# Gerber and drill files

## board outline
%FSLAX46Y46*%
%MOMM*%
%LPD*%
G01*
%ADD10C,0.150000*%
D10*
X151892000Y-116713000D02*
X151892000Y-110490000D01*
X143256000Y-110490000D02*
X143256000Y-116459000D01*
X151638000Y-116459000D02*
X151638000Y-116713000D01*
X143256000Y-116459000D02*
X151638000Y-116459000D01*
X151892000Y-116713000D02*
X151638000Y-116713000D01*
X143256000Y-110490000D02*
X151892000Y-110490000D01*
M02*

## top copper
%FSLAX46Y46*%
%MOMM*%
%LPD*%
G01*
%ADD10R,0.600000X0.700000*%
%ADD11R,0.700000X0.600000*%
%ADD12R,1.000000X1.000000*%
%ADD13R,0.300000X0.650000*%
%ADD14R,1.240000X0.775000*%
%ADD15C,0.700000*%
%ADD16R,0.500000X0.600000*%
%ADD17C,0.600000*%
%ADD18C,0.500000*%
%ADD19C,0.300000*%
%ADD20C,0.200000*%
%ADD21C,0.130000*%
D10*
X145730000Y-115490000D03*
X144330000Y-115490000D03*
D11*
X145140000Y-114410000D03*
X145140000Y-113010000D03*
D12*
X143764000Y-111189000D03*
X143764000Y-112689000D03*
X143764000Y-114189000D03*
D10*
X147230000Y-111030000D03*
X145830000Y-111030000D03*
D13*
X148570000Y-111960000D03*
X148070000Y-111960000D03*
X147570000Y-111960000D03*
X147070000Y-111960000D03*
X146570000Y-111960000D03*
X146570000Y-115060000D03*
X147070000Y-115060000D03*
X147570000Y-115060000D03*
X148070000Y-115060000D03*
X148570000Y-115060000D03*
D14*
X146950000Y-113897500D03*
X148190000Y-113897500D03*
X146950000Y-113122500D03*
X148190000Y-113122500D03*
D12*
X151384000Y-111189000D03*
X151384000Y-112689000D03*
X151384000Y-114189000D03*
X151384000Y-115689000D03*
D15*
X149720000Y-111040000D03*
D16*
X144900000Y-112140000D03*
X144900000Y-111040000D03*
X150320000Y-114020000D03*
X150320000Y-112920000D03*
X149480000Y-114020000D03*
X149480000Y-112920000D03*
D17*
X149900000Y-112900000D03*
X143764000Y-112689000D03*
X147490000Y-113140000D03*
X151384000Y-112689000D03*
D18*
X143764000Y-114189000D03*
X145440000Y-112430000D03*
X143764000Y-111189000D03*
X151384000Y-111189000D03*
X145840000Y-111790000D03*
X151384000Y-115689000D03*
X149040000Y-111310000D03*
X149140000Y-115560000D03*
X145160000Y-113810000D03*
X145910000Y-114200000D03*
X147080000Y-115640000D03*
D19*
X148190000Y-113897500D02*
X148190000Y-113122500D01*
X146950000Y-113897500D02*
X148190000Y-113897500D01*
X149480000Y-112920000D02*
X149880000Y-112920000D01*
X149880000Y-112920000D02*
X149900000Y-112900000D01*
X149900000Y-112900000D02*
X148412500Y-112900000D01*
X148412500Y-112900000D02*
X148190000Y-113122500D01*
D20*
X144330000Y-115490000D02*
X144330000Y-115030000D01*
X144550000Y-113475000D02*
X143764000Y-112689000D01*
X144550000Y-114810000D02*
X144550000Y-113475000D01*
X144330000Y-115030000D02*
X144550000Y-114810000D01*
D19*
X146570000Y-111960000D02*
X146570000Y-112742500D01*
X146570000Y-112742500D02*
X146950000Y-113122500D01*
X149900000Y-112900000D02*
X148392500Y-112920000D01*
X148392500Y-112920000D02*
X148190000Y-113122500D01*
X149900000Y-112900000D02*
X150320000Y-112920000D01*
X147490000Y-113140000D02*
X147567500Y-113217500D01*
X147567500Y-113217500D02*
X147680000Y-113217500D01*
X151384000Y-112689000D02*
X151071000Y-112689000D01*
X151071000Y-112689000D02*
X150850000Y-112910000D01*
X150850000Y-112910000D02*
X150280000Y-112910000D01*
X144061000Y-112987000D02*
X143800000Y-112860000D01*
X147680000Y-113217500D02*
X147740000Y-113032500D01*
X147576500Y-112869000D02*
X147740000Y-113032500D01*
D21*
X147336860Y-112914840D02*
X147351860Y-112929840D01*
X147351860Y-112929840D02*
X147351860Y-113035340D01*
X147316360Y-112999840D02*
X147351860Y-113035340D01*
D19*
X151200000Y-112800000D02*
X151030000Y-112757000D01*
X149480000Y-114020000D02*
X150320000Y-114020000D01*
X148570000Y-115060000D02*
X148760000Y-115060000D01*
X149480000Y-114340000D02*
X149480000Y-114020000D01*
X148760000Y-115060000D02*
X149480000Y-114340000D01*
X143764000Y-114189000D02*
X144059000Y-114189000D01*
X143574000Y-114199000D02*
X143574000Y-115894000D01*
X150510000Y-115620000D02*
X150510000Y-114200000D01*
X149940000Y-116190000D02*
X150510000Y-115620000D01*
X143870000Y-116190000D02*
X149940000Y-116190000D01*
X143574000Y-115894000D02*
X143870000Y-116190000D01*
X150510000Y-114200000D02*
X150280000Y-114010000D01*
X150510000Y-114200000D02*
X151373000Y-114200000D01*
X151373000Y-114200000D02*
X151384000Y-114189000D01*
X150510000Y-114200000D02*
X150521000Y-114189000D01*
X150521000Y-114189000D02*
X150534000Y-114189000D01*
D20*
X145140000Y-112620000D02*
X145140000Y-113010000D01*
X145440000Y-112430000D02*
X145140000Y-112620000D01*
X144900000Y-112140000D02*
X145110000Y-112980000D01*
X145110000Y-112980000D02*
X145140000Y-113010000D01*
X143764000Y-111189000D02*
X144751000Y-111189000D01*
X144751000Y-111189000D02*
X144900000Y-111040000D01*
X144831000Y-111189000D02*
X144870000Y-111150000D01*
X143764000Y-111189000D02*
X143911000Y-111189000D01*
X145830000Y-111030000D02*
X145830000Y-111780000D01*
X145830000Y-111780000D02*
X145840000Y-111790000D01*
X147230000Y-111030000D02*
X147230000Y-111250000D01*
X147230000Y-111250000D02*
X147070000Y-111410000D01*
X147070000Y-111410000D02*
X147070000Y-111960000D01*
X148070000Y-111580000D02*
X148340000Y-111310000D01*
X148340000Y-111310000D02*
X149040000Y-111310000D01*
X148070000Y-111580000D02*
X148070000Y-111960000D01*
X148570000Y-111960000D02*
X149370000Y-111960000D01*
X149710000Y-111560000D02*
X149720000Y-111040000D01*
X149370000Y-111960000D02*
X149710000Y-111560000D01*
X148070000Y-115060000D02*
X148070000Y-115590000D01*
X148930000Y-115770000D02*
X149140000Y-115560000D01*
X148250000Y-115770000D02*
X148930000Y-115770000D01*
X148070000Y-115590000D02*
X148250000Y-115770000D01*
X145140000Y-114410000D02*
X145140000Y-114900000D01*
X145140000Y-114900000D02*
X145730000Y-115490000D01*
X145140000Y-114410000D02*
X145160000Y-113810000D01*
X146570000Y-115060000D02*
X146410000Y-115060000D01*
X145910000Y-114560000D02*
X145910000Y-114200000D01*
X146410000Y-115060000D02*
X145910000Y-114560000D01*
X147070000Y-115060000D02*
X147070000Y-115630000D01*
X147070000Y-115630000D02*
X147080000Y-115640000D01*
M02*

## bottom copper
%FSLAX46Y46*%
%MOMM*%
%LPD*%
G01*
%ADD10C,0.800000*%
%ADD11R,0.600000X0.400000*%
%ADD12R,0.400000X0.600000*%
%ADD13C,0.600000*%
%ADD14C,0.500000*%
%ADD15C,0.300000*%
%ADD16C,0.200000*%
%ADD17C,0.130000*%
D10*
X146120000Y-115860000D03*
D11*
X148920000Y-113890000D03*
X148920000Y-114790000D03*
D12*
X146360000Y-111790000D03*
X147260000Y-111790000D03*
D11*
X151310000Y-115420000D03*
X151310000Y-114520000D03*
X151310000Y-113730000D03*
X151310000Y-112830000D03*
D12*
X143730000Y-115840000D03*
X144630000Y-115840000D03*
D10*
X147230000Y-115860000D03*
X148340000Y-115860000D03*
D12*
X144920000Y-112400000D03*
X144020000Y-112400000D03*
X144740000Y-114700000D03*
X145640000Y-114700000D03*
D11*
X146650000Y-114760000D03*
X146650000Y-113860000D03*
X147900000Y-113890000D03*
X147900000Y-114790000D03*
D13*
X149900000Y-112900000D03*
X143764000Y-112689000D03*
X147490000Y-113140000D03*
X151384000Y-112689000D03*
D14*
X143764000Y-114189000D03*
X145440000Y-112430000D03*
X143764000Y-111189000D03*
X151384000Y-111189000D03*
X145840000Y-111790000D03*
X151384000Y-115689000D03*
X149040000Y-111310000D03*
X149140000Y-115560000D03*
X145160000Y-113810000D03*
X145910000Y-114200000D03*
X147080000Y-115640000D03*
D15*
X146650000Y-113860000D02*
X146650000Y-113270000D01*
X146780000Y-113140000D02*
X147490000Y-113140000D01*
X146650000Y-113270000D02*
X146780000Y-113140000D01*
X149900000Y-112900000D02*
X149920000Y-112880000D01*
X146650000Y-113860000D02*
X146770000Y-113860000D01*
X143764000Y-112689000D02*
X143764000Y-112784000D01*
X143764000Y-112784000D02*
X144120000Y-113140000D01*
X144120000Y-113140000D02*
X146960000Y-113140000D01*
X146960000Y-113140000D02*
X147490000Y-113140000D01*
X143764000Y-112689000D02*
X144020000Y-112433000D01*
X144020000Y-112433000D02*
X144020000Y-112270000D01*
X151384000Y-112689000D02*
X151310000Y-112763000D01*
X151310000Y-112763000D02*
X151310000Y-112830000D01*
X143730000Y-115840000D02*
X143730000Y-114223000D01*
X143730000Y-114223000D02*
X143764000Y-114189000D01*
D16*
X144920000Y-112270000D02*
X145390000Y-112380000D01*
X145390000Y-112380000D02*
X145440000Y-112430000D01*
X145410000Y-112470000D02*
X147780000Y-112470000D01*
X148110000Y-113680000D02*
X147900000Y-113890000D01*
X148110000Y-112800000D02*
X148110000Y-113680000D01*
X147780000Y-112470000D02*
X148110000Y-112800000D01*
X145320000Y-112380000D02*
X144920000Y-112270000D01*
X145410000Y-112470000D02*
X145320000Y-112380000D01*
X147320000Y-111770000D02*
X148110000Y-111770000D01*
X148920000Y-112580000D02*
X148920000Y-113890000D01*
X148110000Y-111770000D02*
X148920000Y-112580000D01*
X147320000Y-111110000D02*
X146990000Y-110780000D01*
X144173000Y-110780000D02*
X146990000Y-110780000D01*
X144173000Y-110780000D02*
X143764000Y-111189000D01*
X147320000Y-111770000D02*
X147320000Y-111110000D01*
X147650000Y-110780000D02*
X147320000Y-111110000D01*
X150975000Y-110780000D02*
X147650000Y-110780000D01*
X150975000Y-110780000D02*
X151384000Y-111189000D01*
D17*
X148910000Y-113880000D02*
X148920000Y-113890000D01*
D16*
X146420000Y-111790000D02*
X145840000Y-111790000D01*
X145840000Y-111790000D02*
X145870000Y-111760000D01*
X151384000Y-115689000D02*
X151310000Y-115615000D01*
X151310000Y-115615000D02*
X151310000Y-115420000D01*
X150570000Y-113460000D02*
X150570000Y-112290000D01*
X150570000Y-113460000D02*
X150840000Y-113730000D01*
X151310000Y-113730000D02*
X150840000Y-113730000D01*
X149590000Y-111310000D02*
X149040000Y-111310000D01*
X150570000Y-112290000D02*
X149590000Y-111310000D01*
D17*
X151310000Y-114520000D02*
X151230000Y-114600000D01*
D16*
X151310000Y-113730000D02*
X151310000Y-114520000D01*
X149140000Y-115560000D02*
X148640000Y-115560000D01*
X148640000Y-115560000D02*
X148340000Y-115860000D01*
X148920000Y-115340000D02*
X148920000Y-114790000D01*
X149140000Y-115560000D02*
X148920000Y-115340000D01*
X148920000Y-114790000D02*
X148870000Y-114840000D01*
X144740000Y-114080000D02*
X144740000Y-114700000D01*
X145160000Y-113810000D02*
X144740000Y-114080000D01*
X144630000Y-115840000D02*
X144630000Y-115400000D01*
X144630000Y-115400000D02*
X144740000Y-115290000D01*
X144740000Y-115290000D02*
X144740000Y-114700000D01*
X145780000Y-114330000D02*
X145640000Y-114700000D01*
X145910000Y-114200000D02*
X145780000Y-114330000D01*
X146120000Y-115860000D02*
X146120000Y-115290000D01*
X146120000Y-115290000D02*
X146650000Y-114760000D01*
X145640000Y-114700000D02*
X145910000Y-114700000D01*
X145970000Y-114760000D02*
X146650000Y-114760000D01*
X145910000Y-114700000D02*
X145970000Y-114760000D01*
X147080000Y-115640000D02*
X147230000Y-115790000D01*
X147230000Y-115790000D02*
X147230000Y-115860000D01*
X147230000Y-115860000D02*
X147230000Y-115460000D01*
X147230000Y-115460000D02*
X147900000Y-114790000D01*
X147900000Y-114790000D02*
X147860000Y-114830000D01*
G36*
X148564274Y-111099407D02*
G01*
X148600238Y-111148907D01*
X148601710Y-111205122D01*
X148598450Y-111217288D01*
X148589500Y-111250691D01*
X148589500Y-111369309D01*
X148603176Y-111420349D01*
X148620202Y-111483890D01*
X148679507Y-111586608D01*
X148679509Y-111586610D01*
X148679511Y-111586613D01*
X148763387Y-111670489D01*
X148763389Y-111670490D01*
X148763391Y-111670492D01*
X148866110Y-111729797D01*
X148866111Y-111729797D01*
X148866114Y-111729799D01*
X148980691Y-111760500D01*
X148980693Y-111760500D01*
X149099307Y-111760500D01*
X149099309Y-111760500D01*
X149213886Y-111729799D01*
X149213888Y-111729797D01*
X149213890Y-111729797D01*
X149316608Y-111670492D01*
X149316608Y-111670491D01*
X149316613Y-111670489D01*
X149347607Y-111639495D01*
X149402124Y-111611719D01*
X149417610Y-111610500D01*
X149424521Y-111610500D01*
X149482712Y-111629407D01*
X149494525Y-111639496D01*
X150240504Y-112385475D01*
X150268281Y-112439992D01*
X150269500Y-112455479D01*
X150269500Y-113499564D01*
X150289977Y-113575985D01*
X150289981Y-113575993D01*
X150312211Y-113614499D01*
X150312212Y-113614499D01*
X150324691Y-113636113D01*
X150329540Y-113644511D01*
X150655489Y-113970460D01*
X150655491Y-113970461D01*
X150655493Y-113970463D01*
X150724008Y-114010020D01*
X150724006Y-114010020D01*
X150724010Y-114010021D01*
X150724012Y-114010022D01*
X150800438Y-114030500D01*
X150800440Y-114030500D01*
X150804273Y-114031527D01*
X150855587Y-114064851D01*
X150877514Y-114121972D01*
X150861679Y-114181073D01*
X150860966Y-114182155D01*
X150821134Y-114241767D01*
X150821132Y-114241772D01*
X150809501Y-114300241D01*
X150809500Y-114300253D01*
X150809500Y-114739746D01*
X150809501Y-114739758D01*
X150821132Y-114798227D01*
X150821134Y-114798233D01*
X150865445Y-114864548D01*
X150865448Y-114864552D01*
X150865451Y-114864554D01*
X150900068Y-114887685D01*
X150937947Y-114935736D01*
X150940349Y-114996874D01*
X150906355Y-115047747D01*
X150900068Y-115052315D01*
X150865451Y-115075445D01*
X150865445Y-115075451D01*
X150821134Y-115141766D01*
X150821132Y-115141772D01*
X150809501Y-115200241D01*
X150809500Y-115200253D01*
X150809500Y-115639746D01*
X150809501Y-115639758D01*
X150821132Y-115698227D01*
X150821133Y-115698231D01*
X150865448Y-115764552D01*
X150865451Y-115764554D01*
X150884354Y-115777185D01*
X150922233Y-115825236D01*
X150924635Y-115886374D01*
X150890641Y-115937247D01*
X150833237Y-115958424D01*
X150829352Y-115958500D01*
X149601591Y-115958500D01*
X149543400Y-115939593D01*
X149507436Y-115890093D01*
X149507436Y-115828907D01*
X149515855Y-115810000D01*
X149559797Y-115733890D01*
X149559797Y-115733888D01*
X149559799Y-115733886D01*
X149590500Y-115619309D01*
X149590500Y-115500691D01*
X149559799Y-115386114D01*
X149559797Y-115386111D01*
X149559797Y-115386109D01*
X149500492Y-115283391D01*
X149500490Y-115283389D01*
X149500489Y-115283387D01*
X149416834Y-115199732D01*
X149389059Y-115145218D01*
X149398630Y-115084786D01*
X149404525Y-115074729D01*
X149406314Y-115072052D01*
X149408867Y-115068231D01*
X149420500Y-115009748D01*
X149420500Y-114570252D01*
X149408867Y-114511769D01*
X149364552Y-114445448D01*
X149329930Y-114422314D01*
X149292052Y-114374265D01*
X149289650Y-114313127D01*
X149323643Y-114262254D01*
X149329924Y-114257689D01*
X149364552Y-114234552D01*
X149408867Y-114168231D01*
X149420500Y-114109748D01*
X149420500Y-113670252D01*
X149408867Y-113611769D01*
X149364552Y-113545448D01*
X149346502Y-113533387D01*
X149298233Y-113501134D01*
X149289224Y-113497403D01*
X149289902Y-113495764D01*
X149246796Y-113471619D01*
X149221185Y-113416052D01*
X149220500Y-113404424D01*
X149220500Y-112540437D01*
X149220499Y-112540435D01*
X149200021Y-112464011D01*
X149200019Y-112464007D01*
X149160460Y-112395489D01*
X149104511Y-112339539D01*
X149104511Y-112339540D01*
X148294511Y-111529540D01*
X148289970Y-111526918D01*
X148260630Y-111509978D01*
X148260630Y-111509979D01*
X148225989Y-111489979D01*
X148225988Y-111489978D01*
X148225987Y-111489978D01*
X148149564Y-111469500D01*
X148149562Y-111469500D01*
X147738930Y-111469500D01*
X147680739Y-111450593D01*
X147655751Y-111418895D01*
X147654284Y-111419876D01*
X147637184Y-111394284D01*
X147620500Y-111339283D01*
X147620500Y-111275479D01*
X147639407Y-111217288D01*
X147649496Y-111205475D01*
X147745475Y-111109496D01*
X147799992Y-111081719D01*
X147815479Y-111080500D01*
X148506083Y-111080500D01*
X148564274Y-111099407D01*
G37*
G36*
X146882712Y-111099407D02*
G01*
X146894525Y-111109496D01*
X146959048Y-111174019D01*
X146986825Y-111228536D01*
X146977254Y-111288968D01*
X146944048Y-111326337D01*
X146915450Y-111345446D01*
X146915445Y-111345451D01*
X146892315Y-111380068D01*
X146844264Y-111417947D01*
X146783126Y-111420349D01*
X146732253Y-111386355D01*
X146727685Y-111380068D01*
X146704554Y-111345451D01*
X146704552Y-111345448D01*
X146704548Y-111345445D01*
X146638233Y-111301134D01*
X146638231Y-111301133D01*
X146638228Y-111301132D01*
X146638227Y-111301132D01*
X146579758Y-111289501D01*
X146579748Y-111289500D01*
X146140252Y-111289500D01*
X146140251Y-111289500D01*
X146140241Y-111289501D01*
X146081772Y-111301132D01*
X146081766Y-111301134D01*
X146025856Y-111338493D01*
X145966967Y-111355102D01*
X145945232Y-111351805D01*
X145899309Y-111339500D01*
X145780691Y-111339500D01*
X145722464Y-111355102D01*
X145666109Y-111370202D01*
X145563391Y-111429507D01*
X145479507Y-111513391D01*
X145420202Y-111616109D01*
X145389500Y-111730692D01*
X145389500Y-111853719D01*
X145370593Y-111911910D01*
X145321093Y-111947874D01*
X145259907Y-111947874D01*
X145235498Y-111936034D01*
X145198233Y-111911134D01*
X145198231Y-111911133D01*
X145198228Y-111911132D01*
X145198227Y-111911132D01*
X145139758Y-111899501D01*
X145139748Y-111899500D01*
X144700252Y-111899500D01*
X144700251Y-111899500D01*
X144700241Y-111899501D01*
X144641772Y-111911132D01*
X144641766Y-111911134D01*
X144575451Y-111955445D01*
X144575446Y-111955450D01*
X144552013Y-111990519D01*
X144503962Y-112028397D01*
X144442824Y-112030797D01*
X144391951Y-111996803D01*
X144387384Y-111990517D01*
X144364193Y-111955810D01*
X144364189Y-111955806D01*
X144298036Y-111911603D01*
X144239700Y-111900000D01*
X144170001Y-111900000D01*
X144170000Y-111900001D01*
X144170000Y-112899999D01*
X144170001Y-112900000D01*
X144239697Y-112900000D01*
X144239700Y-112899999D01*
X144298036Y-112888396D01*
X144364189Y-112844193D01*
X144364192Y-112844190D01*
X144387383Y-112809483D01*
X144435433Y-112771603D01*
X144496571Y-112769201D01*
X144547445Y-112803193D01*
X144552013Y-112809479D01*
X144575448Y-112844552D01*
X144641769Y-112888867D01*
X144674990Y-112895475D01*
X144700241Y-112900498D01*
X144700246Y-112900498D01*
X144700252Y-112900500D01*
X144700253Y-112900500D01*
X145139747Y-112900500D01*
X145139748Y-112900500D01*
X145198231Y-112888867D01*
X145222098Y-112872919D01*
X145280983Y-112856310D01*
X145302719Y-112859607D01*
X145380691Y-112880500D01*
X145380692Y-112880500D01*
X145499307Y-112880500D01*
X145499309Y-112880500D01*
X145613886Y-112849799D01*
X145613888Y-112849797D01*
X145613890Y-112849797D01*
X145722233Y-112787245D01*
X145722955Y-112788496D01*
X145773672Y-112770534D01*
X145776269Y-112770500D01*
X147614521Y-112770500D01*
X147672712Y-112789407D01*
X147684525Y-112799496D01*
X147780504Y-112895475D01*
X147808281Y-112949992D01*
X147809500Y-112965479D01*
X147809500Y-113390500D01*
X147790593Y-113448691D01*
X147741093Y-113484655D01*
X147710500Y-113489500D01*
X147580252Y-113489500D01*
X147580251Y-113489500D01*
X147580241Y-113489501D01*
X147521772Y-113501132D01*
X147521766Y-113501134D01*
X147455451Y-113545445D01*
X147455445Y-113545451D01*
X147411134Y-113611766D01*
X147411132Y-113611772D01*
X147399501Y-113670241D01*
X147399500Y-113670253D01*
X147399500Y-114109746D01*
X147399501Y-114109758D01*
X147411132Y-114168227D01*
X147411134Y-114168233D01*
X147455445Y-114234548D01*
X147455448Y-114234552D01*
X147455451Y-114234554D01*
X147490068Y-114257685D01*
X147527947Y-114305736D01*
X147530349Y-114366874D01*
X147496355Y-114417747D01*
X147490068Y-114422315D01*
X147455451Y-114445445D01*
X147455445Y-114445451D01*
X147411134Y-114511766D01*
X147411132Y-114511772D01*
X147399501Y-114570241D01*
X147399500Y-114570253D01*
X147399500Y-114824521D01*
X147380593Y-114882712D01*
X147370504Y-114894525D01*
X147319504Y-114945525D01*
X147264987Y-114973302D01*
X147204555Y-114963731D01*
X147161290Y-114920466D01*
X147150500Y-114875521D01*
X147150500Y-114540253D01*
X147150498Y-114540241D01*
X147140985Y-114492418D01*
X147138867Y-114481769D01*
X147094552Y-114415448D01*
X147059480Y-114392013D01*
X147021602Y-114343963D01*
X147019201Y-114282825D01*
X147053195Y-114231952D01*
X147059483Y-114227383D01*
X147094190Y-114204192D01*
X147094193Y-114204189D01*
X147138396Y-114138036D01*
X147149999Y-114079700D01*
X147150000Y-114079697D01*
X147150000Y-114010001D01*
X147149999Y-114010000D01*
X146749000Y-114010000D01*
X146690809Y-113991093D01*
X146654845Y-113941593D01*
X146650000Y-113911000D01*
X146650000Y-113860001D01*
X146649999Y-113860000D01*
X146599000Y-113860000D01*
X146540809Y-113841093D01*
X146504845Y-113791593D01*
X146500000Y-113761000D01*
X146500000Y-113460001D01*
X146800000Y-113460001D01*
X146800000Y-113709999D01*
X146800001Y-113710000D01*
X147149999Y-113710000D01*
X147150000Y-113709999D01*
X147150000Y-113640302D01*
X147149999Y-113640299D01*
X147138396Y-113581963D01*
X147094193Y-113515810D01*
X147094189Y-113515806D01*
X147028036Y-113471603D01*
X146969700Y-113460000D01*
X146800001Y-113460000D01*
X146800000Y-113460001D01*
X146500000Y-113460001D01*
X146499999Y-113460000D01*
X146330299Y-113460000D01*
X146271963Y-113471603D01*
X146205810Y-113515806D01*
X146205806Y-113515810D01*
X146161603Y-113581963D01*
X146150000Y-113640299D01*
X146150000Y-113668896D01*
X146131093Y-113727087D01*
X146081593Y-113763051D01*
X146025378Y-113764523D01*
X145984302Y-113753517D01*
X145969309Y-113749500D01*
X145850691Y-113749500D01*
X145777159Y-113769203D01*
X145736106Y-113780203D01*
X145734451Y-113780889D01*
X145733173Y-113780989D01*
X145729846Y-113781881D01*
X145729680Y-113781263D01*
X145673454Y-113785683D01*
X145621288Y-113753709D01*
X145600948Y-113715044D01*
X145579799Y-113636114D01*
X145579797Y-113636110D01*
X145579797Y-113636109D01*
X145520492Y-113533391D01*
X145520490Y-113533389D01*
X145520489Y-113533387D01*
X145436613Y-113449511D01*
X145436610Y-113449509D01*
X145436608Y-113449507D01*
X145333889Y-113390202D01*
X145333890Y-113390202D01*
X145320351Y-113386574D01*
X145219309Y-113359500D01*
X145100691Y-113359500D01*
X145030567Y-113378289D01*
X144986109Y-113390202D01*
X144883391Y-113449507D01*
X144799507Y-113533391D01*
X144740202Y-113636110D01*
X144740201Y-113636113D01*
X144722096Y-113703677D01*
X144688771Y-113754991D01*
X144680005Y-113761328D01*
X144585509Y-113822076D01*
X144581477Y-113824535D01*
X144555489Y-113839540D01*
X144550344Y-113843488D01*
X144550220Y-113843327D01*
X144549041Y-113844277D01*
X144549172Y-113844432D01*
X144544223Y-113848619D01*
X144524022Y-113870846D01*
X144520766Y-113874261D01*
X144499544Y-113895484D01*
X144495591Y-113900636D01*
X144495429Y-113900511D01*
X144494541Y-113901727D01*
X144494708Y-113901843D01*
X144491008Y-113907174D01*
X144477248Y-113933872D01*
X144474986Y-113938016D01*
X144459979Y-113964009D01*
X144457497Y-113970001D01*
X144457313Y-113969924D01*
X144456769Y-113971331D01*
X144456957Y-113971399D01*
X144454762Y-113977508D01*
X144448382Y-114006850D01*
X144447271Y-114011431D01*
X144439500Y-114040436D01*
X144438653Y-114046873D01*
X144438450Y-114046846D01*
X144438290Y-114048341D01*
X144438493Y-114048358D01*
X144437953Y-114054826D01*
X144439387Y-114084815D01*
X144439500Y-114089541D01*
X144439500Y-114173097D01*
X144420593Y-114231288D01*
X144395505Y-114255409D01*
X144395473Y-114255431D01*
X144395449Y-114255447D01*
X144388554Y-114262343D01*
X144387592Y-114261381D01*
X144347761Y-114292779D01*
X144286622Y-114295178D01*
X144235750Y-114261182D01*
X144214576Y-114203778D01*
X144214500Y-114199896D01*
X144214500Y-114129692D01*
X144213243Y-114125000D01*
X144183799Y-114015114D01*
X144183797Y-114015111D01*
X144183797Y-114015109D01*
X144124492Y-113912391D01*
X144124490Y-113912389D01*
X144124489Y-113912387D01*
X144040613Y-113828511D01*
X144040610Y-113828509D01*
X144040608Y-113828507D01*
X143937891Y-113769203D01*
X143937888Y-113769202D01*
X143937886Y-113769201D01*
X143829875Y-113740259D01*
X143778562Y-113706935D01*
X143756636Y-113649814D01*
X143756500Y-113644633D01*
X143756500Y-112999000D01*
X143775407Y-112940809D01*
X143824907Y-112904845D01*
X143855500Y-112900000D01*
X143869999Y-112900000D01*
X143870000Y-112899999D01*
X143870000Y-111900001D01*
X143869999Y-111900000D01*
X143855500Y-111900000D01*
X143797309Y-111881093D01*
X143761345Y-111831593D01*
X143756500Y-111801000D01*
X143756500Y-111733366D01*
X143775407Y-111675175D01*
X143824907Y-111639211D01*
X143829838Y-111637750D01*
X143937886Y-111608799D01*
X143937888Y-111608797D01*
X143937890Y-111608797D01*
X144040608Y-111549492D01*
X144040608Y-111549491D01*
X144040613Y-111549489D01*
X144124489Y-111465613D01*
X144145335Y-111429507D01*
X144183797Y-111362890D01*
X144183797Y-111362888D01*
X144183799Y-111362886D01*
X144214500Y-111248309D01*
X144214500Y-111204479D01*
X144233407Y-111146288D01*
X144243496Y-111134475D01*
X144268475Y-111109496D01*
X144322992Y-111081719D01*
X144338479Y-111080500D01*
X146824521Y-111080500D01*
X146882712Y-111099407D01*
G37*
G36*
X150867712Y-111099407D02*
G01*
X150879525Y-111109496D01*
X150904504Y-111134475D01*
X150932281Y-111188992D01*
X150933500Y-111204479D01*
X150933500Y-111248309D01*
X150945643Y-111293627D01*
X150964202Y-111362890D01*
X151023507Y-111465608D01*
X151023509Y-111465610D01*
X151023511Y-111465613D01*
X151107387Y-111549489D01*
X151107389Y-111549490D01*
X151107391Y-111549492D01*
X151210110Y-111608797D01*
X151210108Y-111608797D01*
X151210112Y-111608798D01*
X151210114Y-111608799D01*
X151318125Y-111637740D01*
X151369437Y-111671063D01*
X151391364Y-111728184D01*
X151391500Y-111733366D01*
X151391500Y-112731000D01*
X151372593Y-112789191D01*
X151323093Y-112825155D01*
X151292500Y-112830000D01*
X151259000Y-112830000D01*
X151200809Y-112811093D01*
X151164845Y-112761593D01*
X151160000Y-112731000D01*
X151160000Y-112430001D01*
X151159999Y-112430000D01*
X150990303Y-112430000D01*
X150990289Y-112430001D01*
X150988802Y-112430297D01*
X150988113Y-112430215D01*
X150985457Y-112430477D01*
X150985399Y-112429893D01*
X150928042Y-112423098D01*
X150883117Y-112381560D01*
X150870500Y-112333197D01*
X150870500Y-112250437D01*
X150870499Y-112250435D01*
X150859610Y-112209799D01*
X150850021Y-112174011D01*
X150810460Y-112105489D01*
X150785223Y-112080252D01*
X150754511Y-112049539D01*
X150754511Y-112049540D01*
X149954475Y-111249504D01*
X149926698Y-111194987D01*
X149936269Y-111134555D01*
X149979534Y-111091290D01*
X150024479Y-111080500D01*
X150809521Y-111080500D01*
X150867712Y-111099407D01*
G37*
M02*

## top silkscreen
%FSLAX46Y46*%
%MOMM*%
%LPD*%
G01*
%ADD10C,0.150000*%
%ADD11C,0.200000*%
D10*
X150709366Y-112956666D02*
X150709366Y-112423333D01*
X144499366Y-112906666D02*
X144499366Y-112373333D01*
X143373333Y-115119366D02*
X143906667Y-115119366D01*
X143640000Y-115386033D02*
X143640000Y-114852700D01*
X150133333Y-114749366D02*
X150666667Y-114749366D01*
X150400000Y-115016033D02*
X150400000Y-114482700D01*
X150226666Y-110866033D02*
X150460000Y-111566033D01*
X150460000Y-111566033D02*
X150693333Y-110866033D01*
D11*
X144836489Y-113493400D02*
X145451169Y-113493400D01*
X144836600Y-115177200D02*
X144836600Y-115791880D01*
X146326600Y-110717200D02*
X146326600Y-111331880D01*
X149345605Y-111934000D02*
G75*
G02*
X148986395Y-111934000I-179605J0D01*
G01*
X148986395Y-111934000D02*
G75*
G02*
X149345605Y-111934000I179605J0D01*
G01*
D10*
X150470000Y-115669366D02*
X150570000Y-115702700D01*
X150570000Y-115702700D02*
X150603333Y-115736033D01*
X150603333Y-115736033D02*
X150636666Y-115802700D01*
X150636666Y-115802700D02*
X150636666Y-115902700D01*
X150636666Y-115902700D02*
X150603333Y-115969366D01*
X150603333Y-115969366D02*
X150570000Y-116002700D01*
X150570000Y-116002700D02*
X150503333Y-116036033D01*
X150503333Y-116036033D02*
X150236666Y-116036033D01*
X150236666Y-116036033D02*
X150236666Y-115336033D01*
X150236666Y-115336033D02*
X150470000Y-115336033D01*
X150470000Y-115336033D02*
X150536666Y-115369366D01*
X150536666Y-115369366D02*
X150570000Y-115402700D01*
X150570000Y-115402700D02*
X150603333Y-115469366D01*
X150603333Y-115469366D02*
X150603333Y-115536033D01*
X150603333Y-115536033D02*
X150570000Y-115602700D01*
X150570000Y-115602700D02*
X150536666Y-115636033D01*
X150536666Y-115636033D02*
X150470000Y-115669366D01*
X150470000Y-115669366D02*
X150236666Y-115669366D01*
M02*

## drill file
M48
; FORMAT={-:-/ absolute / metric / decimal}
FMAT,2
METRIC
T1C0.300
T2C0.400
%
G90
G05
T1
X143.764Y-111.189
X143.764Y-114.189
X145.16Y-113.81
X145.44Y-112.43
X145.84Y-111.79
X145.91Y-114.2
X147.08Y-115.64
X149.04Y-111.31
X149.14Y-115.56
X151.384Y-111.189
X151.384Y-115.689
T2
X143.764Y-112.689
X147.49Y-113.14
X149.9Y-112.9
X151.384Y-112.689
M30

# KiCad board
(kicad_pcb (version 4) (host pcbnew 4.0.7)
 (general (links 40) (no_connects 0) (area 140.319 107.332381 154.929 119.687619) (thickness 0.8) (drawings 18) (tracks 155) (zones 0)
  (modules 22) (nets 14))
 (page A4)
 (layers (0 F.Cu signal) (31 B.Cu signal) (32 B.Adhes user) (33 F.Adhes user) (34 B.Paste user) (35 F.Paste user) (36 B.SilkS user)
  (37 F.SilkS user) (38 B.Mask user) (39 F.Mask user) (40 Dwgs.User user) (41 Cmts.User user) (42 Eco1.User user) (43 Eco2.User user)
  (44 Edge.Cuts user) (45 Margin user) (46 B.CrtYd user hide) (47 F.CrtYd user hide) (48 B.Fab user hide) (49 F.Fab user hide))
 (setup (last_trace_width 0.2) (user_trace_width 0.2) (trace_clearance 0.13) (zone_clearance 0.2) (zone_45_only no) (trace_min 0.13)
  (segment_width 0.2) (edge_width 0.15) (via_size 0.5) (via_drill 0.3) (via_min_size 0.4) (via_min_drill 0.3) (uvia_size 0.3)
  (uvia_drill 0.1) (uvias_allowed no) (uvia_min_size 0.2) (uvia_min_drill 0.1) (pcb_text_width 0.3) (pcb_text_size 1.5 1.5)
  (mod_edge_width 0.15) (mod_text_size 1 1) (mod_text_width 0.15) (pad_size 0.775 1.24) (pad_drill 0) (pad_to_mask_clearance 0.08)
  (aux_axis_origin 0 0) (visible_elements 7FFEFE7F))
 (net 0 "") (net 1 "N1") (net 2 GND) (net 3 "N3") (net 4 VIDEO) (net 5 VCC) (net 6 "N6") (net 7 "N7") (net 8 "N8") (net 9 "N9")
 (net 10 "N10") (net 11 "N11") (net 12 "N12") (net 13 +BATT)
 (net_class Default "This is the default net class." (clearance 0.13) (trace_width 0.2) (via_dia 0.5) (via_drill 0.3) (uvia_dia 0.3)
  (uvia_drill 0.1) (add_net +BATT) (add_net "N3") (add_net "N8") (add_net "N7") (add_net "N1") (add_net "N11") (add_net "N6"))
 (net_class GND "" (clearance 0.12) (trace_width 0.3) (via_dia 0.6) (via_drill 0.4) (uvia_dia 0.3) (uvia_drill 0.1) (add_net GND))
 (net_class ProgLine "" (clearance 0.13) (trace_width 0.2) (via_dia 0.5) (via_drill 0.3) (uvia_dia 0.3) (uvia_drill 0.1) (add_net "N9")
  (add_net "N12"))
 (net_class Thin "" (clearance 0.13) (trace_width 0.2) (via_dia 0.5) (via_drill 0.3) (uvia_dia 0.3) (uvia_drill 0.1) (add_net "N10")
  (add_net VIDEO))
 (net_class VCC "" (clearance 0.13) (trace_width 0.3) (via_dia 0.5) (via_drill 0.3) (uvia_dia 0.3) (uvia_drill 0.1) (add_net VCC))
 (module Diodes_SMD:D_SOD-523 (layer F.Cu) (at 145.03 115.49)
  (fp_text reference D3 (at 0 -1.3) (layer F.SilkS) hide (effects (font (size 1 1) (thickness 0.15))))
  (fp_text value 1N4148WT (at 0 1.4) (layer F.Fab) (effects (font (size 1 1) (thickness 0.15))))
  (pad 2 smd rect (at 0.7 0 180) (size 0.6 0.7) (layers F.Cu F.Paste F.Mask) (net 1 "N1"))
  (pad 1 smd rect (at -0.7 0 180) (size 0.6 0.7) (layers F.Cu F.Paste F.Mask) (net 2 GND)))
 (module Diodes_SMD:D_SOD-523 (layer F.Cu) (at 145.14 113.71 270)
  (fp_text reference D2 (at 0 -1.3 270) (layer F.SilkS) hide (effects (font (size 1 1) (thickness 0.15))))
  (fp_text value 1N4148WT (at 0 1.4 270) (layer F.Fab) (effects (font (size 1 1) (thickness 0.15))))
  (pad 2 smd rect (at 0.7 0 90) (size 0.6 0.7) (layers F.Cu F.Paste F.Mask) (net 1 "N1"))
  (pad 1 smd rect (at -0.7 0 90) (size 0.6 0.7) (layers F.Cu F.Paste F.Mask) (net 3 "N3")))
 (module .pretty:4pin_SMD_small (layer F.Cu) (at 143.764 115.189 90)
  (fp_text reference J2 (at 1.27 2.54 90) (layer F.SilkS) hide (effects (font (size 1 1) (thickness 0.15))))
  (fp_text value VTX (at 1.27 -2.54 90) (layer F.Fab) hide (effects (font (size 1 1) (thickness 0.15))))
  (pad 4 smd rect (at 4 0 90) (size 1 1) (layers F.Cu F.Paste F.Mask) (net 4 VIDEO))
  (pad 3 smd rect (at 2.5 0 90) (size 1 1) (layers F.Cu F.Paste F.Mask) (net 2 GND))
  (pad 2 smd rect (at 1 0 90) (size 1 1) (layers F.Cu F.Paste F.Mask) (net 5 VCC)))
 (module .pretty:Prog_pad (layer B.Cu) (at 146.12 115.86)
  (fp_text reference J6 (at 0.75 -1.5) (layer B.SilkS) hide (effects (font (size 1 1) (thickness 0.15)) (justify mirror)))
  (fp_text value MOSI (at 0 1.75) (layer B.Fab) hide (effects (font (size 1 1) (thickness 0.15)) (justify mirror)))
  (pad 1 smd circle (at 0 0) (size 0.8 0.8) (layers B.Cu B.Paste B.Mask) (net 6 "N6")))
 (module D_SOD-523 (layer F.Cu) (at 146.53 111.03)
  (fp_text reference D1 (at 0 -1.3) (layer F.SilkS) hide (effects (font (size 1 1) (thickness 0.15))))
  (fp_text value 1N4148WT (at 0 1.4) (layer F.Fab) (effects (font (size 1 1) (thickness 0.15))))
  (pad 2 smd rect (at 0.7 0 180) (size 0.6 0.7) (layers F.Cu F.Paste F.Mask) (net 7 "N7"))
  (pad 1 smd rect (at -0.7 0 180) (size 0.6 0.7) (layers F.Cu F.Paste F.Mask) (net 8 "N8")))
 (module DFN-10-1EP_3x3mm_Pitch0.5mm (layer F.Cu) (at 147.57 113.51 270)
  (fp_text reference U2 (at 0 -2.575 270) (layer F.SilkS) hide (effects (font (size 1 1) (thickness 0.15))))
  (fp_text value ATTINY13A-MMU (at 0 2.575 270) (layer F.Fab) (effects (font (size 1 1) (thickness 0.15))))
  (pad 1 smd rect (at -1.55 -1 270) (size 0.65 0.3) (layers F.Cu F.Paste F.Mask) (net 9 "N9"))
  (pad 2 smd rect (at -1.55 -0.5 270) (size 0.65 0.3) (layers F.Cu F.Paste F.Mask) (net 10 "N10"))
  (pad 3 smd rect (at -1.55 0 270) (size 0.65 0.3) (layers F.Cu F.Paste F.Mask))
  (pad 4 smd rect (at -1.55 0.5 270) (size 0.65 0.3) (layers F.Cu F.Paste F.Mask) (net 7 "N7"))
  (pad 5 smd rect (at -1.55 1 270) (size 0.65 0.3) (layers F.Cu F.Paste F.Mask) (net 2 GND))
  (pad 6 smd rect (at 1.55 1 270) (size 0.65 0.3) (layers F.Cu F.Paste F.Mask) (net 6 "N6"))
  (pad 7 smd rect (at 1.55 0.5 270) (size 0.65 0.3) (layers F.Cu F.Paste F.Mask) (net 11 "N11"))
  (pad 8 smd rect (at 1.55 0 270) (size 0.65 0.3) (layers F.Cu F.Paste F.Mask))
  (pad 9 smd rect (at 1.55 -0.5 270) (size 0.65 0.3) (layers F.Cu F.Paste F.Mask) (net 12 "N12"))
  (pad 10 smd rect (at 1.55 -1 270) (size 0.65 0.3) (layers F.Cu F.Paste F.Mask) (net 5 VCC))
  (pad 5 smd rect (at 0.3875 0.62 270) (size 0.775 1.24) (layers F.Cu F.Paste F.Mask) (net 2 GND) (solder_paste_margin_ratio -0.2))
  (pad 5 smd rect (at 0.3875 -0.62 270) (size 0.775 1.24) (layers F.Cu F.Paste F.Mask) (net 2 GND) (solder_paste_margin_ratio -0.2))
  (pad 5 smd rect (at -0.3875 0.62 270) (size 0.775 1.24) (layers F.Cu F.Paste F.Mask) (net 2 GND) (solder_paste_margin_ratio -0.2))
  (pad 5 smd rect (at -0.3875 -0.62 270) (size 0.775 1.24) (layers F.Cu F.Paste F.Mask) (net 2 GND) (solder_paste_margin_ratio -0.2)))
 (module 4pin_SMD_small (layer F.Cu) (at 151.384 115.189 90)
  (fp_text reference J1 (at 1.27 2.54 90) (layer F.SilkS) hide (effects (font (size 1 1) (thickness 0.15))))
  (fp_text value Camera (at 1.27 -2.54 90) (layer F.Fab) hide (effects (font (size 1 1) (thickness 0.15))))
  (pad 4 smd rect (at 4 0 90) (size 1 1) (layers F.Cu F.Paste F.Mask) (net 4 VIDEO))
  (pad 3 smd rect (at 2.5 0 90) (size 1 1) (layers F.Cu F.Paste F.Mask) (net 2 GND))
  (pad 2 smd rect (at 1 0 90) (size 1 1) (layers F.Cu F.Paste F.Mask) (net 5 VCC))
  (pad 1 smd rect (at -0.5 0 90) (size 1 1) (layers F.Cu F.Paste F.Mask) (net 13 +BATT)))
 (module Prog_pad (layer F.Cu) (at 149.72 111.04)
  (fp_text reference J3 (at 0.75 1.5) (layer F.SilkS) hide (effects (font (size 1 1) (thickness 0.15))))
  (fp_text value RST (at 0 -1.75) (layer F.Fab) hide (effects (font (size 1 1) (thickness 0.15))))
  (pad 1 smd circle (at 0 0) (size 0.7 0.7) (layers F.Cu F.Paste F.Mask) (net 9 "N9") (solder_mask_margin 0.02)))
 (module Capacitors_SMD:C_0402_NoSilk (layer F.Cu) (at 144.9 111.59 90)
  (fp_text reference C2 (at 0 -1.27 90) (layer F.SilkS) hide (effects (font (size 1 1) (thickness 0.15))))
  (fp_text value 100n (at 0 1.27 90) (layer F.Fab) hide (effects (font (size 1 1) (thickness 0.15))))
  (pad 1 smd rect (at -0.55 0 90) (size 0.6 0.5) (layers F.Cu F.Paste F.Mask) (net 3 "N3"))
  (pad 2 smd rect (at 0.55 0 90) (size 0.6 0.5) (layers F.Cu F.Paste F.Mask) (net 4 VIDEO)))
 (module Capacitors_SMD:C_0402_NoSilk (layer F.Cu) (at 150.32 113.47 90)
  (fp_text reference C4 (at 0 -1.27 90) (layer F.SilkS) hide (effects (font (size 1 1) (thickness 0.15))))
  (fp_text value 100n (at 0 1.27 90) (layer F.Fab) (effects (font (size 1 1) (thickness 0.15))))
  (pad 1 smd rect (at -0.55 0 90) (size 0.6 0.5) (layers F.Cu F.Paste F.Mask) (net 5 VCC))
  (pad 2 smd rect (at 0.55 0 90) (size 0.6 0.5) (layers F.Cu F.Paste F.Mask) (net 2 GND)))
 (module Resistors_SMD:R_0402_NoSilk (layer B.Cu) (at 148.92 114.34 270)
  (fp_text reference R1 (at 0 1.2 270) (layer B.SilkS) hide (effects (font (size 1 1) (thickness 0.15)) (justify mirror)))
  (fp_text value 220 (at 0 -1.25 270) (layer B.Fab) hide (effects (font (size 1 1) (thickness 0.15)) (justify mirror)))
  (pad 1 smd rect (at -0.45 0 270) (size 0.4 0.6) (layers B.Cu B.Paste B.Mask) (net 4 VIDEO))
  (pad 2 smd rect (at 0.45 0 270) (size 0.4 0.6) (layers B.Cu B.Paste B.Mask) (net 12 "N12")))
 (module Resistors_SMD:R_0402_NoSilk (layer B.Cu) (at 146.81 111.79)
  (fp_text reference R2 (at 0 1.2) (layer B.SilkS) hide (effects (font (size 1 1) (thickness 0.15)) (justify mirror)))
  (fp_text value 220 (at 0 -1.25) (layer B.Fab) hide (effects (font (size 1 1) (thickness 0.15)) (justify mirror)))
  (pad 1 smd rect (at -0.45 0) (size 0.4 0.6) (layers B.Cu B.Paste B.Mask) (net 8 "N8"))
  (pad 2 smd rect (at 0.45 0) (size 0.4 0.6) (layers B.Cu B.Paste B.Mask) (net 4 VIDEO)))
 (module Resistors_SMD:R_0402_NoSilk (layer B.Cu) (at 151.31 114.97 90)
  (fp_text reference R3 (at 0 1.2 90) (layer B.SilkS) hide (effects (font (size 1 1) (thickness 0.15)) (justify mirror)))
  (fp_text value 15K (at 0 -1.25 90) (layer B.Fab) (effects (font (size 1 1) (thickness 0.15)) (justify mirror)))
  (pad 1 smd rect (at -0.45 0 90) (size 0.4 0.6) (layers B.Cu B.Paste B.Mask) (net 13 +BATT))
  (pad 2 smd rect (at 0.45 0 90) (size 0.4 0.6) (layers B.Cu B.Paste B.Mask) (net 10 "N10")))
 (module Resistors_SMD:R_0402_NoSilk (layer B.Cu) (at 151.31 113.28 90)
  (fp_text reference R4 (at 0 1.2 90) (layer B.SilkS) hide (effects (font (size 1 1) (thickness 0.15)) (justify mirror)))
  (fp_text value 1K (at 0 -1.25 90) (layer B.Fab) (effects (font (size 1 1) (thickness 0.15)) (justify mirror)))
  (pad 1 smd rect (at -0.45 0 90) (size 0.4 0.6) (layers B.Cu B.Paste B.Mask) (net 10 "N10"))
  (pad 2 smd rect (at 0.45 0 90) (size 0.4 0.6) (layers B.Cu B.Paste B.Mask) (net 2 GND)))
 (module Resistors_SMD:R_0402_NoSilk (layer B.Cu) (at 144.18 115.84)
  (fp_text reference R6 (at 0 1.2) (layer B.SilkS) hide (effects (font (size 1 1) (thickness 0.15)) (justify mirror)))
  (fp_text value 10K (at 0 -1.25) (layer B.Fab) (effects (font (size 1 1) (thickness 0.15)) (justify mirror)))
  (pad 1 smd rect (at -0.45 0) (size 0.4 0.6) (layers B.Cu B.Paste B.Mask) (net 5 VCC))
  (pad 2 smd rect (at 0.45 0) (size 0.4 0.6) (layers B.Cu B.Paste B.Mask) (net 1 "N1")))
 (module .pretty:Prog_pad (layer B.Cu) (at 147.23 115.86)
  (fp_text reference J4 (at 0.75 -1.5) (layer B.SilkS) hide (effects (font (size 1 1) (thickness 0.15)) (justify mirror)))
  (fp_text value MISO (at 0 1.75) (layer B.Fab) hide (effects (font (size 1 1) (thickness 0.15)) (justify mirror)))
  (pad 1 smd circle (at 0 0) (size 0.8 0.8) (layers B.Cu B.Paste B.Mask) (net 11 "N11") (solder_mask_margin 0.02)))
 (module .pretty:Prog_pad (layer B.Cu) (at 148.34 115.86)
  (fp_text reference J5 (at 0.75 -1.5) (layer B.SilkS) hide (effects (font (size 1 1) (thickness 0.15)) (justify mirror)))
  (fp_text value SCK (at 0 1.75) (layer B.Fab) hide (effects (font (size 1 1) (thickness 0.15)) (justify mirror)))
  (pad 1 smd circle (at 0 0) (size 0.8 0.8) (layers B.Cu B.Paste B.Mask) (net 12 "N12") (solder_mask_margin 0.02)))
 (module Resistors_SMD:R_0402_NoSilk (layer B.Cu) (at 144.47 112.4 180)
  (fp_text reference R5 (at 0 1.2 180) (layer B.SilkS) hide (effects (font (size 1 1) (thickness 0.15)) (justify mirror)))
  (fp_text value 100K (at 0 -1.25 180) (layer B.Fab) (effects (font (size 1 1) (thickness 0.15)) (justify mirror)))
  (pad 1 smd rect (at -0.45 0 180) (size 0.4 0.6) (layers B.Cu B.Paste B.Mask) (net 3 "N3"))
  (pad 2 smd rect (at 0.45 0 180) (size 0.4 0.6) (layers B.Cu B.Paste B.Mask) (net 2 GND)))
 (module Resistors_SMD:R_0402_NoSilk (layer B.Cu) (at 145.19 114.7)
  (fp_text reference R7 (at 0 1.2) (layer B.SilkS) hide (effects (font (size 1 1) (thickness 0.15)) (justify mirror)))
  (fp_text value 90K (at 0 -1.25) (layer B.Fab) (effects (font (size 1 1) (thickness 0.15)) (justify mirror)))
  (pad 1 smd rect (at -0.45 0) (size 0.4 0.6) (layers B.Cu B.Paste B.Mask) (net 1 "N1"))
  (pad 2 smd rect (at 0.45 0) (size 0.4 0.6) (layers B.Cu B.Paste B.Mask) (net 6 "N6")))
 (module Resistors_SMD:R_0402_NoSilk (layer B.Cu) (at 146.65 114.31 90)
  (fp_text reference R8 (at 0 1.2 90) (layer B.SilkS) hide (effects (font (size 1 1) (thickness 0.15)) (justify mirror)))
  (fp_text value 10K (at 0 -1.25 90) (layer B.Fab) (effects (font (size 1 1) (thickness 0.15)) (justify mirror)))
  (pad 1 smd rect (at -0.45 0 90) (size 0.4 0.6) (layers B.Cu B.Paste B.Mask) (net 6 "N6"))
  (pad 2 smd rect (at 0.45 0 90) (size 0.4 0.6) (layers B.Cu B.Paste B.Mask) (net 2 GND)))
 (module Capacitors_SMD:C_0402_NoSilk (layer F.Cu) (at 149.48 113.47 90)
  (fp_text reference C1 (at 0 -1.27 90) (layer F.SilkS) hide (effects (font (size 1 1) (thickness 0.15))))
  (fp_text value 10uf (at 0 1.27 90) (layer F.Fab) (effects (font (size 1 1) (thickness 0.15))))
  (pad 1 smd rect (at -0.55 0 90) (size 0.6 0.5) (layers F.Cu F.Paste F.Mask) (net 5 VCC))
  (pad 2 smd rect (at 0.55 0 90) (size 0.6 0.5) (layers F.Cu F.Paste F.Mask) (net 2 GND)))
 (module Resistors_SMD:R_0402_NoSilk (layer B.Cu) (at 147.9 114.34 270)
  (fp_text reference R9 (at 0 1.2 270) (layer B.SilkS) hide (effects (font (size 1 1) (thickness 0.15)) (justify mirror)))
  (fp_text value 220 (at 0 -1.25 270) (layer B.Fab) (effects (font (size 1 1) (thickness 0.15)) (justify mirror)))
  (pad 1 smd rect (at -0.45 0 270) (size 0.4 0.6) (layers B.Cu B.Paste B.Mask) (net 3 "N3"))
  (pad 2 smd rect (at 0.45 0 270) (size 0.4 0.6) (layers B.Cu B.Paste B.Mask) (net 11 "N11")))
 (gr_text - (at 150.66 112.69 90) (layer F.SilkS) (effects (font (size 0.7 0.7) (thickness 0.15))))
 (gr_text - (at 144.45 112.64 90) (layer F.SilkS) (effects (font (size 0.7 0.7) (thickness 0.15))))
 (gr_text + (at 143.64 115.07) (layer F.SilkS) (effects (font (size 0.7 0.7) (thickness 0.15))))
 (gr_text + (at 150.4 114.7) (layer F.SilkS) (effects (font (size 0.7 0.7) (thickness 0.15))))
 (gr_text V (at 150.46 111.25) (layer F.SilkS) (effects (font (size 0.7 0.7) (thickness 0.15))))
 (gr_line (start 144.836489 113.4934) (end 145.451169 113.4934) (angle 90) (layer F.SilkS) (width 0.2))
 (gr_line (start 144.8366 115.1772) (end 144.8366 115.79188) (angle 90) (layer F.SilkS) (width 0.2))
 (gr_line (start 146.3266 110.7172) (end 146.3266 111.33188) (angle 90) (layer F.SilkS) (width 0.2))
 (gr_line (start 151.892 116.713) (end 151.892 110.49) (angle 90) (layer Edge.Cuts) (width 0.15))
 (gr_line (start 143.256 110.49) (end 143.256 116.459) (angle 90) (layer Edge.Cuts) (width 0.15))
 (gr_line (start 151.638 116.459) (end 151.638 116.713) (angle 90) (layer Edge.Cuts) (width 0.15))
 (gr_line (start 143.256 116.459) (end 151.638 116.459) (angle 90) (layer Edge.Cuts) (width 0.15))
 (gr_line (start 151.892 116.713) (end 151.638 116.713) (angle 90) (layer Edge.Cuts) (width 0.15))
 (gr_circle (center 149.166 111.934) (end 149.039 111.807) (layer F.SilkS) (width 0.2))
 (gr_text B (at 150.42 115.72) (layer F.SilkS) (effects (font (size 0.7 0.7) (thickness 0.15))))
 (gr_line (start 143.256 110.49) (end 151.892 110.49) (angle 90) (layer Edge.Cuts) (width 0.15))
 (segment (start 148.19 113.8975) (end 148.19 113.1225) (width 0.3) (layer F.Cu) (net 2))
 (segment (start 146.95 113.8975) (end 148.19 113.8975) (width 0.3) (layer F.Cu) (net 2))
 (segment (start 146.65 113.86) (end 146.65 113.27) (width 0.3) (layer B.Cu) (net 2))
 (segment (start 146.78 113.14) (end 147.49 113.14) (width 0.3) (layer B.Cu) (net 2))
 (segment (start 146.65 113.27) (end 146.78 113.14) (width 0.3) (layer B.Cu) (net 2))
 (segment (start 149.48 112.92) (end 149.88 112.92) (width 0.3) (layer F.Cu) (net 2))
 (segment (start 149.88 112.92) (end 149.9 112.9) (width 0.3) (layer F.Cu) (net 2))
 (segment (start 149.9 112.9) (end 148.4125 112.9) (width 0.3) (layer F.Cu) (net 2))
 (segment (start 148.4125 112.9) (end 148.19 113.1225) (width 0.3) (layer F.Cu) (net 2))
 (via (at 149.9 112.9) (size 0.6) (drill 0.4) (layers F.Cu B.Cu) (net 2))
 (segment (start 149.9 112.9) (end 149.92 112.88) (width 0.3) (layer B.Cu) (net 2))
 (segment (start 144.33 115.49) (end 144.33 115.03) (width 0.2) (layer F.Cu) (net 2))
 (segment (start 144.55 113.475) (end 143.764 112.689) (width 0.2) (layer F.Cu) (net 2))
 (segment (start 144.55 114.81) (end 144.55 113.475) (width 0.2) (layer F.Cu) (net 2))
 (segment (start 144.33 115.03) (end 144.55 114.81) (width 0.2) (layer F.Cu) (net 2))
 (segment (start 146.57 111.96) (end 146.57 112.7425) (width 0.3) (layer F.Cu) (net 2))
 (segment (start 146.57 112.7425) (end 146.95 113.1225) (width 0.3) (layer F.Cu) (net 2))
 (segment (start 149.9 112.9) (end 148.3925 112.92) (width 0.3) (layer F.Cu) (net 2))
 (segment (start 148.3925 112.92) (end 148.19 113.1225) (width 0.3) (layer F.Cu) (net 2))
 (segment (start 149.9 112.9) (end 150.32 112.92) (width 0.3) (layer F.Cu) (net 2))
 (segment (start 146.65 113.86) (end 146.77 113.86) (width 0.3) (layer B.Cu) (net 2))
 (via (at 143.764 112.689) (size 0.6) (drill 0.4) (layers F.Cu B.Cu) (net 2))
 (segment (start 143.764 112.689) (end 143.764 112.784) (width 0.3) (layer B.Cu) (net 2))
 (segment (start 143.764 112.784) (end 144.12 113.14) (width 0.3) (layer B.Cu) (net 2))
 (segment (start 144.12 113.14) (end 146.96 113.14) (width 0.3) (layer B.Cu) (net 2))
 (segment (start 146.96 113.14) (end 147.49 113.14) (width 0.3) (layer B.Cu) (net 2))
 (segment (start 147.49 113.14) (end 147.5675 113.2175) (width 0.3) (layer F.Cu) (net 2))
 (via (at 147.49 113.14) (size 0.6) (drill 0.4) (layers F.Cu B.Cu) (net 2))
 (segment (start 147.5675 113.2175) (end 147.68 113.2175) (width 0.3) (layer F.Cu) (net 2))
 (segment (start 143.764 112.689) (end 144.02 112.433) (width 0.3) (layer B.Cu) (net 2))
 (segment (start 144.02 112.433) (end 144.02 112.27) (width 0.3) (layer B.Cu) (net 2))
 (via (at 151.384 112.689) (size 0.6) (drill 0.4) (layers F.Cu B.Cu) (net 2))
 (segment (start 151.384 112.689) (end 151.31 112.763) (width 0.3) (layer B.Cu) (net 2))
 (segment (start 151.31 112.763) (end 151.31 112.83) (width 0.3) (layer B.Cu) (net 2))
 (segment (start 151.384 112.689) (end 151.071 112.689) (width 0.3) (layer F.Cu) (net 2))
 (segment (start 151.071 112.689) (end 150.85 112.91) (width 0.3) (layer F.Cu) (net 2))
 (segment (start 150.85 112.91) (end 150.28 112.91) (width 0.3) (layer F.Cu) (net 2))
 (segment (start 144.061 112.987) (end 143.8 112.86) (width 0.3) (layer F.Cu) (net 2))
 (segment (start 147.68 113.2175) (end 147.74 113.0325) (width 0.3) (layer F.Cu) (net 2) (status 30))
 (segment (start 147.5765 112.869) (end 147.74 113.0325) (width 0.3) (layer F.Cu) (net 2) (status 30))
 (segment (start 147.33686 112.91484) (end 147.35186 112.92984) (width 0.13) (layer F.Cu) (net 2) (status 30))
 (segment (start 147.35186 112.92984) (end 147.35186 113.03534) (width 0.13) (layer F.Cu) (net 2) (status 30))
 (segment (start 147.31636 112.99984) (end 147.35186 113.03534) (width 0.13) (layer F.Cu) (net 2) (status 30))
 (segment (start 151.2 112.8) (end 151.03 112.757) (width 0.3) (layer F.Cu) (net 2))
 (segment (start 149.48 114.02) (end 150.32 114.02) (width 0.3) (layer F.Cu) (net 5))
 (segment (start 148.57 115.06) (end 148.76 115.06) (width 0.3) (layer F.Cu) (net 5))
 (segment (start 149.48 114.34) (end 149.48 114.02) (width 0.3) (layer F.Cu) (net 5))
 (segment (start 148.76 115.06) (end 149.48 114.34) (width 0.3) (layer F.Cu) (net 5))
 (via (at 143.764 114.189) (size 0.5) (drill 0.3) (layers F.Cu B.Cu) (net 5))
 (segment (start 143.73 115.84) (end 143.73 114.223) (width 0.3) (layer B.Cu) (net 5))
 (segment (start 143.73 114.223) (end 143.764 114.189) (width 0.3) (layer B.Cu) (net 5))
 (segment (start 143.764 114.189) (end 144.059 114.189) (width 0.3) (layer F.Cu) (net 5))
 (segment (start 143.574 114.199) (end 143.574 115.894) (width 0.3) (layer F.Cu) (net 5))
 (segment (start 150.51 115.62) (end 150.51 114.2) (width 0.3) (layer F.Cu) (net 5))
 (segment (start 149.94 116.19) (end 150.51 115.62) (width 0.3) (layer F.Cu) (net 5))
 (segment (start 143.87 116.19) (end 149.94 116.19) (width 0.3) (layer F.Cu) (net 5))
 (segment (start 143.574 115.894) (end 143.87 116.19) (width 0.3) (layer F.Cu) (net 5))
 (segment (start 150.51 114.2) (end 150.28 114.01) (width 0.3) (layer F.Cu) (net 5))
 (segment (start 150.51 114.2) (end 151.373 114.2) (width 0.3) (layer F.Cu) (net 5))
 (segment (start 151.373 114.2) (end 151.384 114.189) (width 0.3) (layer F.Cu) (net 5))
 (segment (start 150.51 114.2) (end 150.521 114.189) (width 0.3) (layer F.Cu) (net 5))
 (segment (start 150.521 114.189) (end 150.534 114.189) (width 0.3) (layer F.Cu) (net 5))
 (segment (start 144.92 112.27) (end 145.39 112.38) (width 0.2) (layer B.Cu) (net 3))
 (segment (start 145.14 112.62) (end 145.14 113.01) (width 0.2) (layer F.Cu) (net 3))
 (segment (start 145.44 112.43) (end 145.14 112.62) (width 0.2) (layer F.Cu) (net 3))
 (via (at 145.44 112.43) (size 0.5) (drill 0.3) (layers F.Cu B.Cu) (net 3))
 (segment (start 145.39 112.38) (end 145.44 112.43) (width 0.2) (layer B.Cu) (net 3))
 (segment (start 144.9 112.14) (end 145.11 112.98) (width 0.2) (layer F.Cu) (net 3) (status 20))
 (segment (start 145.11 112.98) (end 145.14 113.01) (width 0.2) (layer F.Cu) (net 3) (status 30))
 (segment (start 145.41 112.47) (end 147.78 112.47) (width 0.2) (layer B.Cu) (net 3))
 (segment (start 148.11 113.68) (end 147.9 113.89) (width 0.2) (layer B.Cu) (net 3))
 (segment (start 148.11 112.8) (end 148.11 113.68) (width 0.2) (layer B.Cu) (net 3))
 (segment (start 147.78 112.47) (end 148.11 112.8) (width 0.2) (layer B.Cu) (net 3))
 (segment (start 145.32 112.38) (end 144.92 112.27) (width 0.2) (layer B.Cu) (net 3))
 (segment (start 145.41 112.47) (end 145.32 112.38) (width 0.2) (layer B.Cu) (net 3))
 (segment (start 143.764 111.189) (end 144.751 111.189) (width 0.2) (layer F.Cu) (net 4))
 (segment (start 144.751 111.189) (end 144.9 111.04) (width 0.2) (layer F.Cu) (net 4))
 (segment (start 147.32 111.77) (end 148.11 111.77) (width 0.2) (layer B.Cu) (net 4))
 (segment (start 148.92 112.58) (end 148.92 113.89) (width 0.2) (layer B.Cu) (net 4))
 (segment (start 148.11 111.77) (end 148.92 112.58) (width 0.2) (layer B.Cu) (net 4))
 (segment (start 144.831 111.189) (end 144.87 111.15) (width 0.2) (layer F.Cu) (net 4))
 (segment (start 143.764 111.189) (end 143.911 111.189) (width 0.2) (layer F.Cu) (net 4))
 (via (at 143.764 111.189) (size 0.5) (drill 0.3) (layers F.Cu B.Cu) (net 4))
 (segment (start 147.32 111.11) (end 146.99 110.78) (width 0.2) (layer B.Cu) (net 4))
 (segment (start 144.173 110.78) (end 146.99 110.78) (width 0.2) (layer B.Cu) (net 4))
 (segment (start 144.173 110.78) (end 143.764 111.189) (width 0.2) (layer B.Cu) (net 4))
 (via (at 151.384 111.189) (size 0.5) (drill 0.3) (layers F.Cu B.Cu) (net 4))
 (segment (start 147.32 111.77) (end 147.32 111.11) (width 0.2) (layer B.Cu) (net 4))
 (segment (start 147.65 110.78) (end 147.32 111.11) (width 0.2) (layer B.Cu) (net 4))
 (segment (start 150.975 110.78) (end 147.65 110.78) (width 0.2) (layer B.Cu) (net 4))
 (segment (start 150.975 110.78) (end 151.384 111.189) (width 0.2) (layer B.Cu) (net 4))
 (segment (start 148.91 113.88) (end 148.92 113.89) (width 0.13) (layer B.Cu) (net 4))
 (segment (start 146.42 111.79) (end 145.84 111.79) (width 0.2) (layer B.Cu) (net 8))
 (segment (start 145.83 111.03) (end 145.83 111.78) (width 0.2) (layer F.Cu) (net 8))
 (segment (start 145.84 111.79) (end 145.87 111.76) (width 0.2) (layer B.Cu) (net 8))
 (via (at 145.84 111.79) (size 0.5) (drill 0.3) (layers F.Cu B.Cu) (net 8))
 (segment (start 145.83 111.78) (end 145.84 111.79) (width 0.2) (layer F.Cu) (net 8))
 (segment (start 147.23 111.03) (end 147.23 111.25) (width 0.2) (layer F.Cu) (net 7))
 (segment (start 147.23 111.25) (end 147.07 111.41) (width 0.2) (layer F.Cu) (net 7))
 (segment (start 147.07 111.41) (end 147.07 111.96) (width 0.2) (layer F.Cu) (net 7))
 (via (at 151.384 115.689) (size 0.5) (drill 0.3) (layers F.Cu B.Cu) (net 13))
 (segment (start 151.384 115.689) (end 151.31 115.615) (width 0.2) (layer B.Cu) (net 13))
 (segment (start 151.31 115.615) (end 151.31 115.42) (width 0.2) (layer B.Cu) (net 13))
 (segment (start 150.57 113.46) (end 150.57 112.29) (width 0.2) (layer B.Cu) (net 10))
 (segment (start 148.07 111.58) (end 148.34 111.31) (width 0.2) (layer F.Cu) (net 10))
 (segment (start 148.34 111.31) (end 149.04 111.31) (width 0.2) (layer F.Cu) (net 10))
 (via (at 149.04 111.31) (size 0.5) (drill 0.3) (layers F.Cu B.Cu) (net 10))
 (segment (start 150.57 113.46) (end 150.84 113.73) (width 0.2) (layer B.Cu) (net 10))
 (segment (start 151.31 113.73) (end 150.84 113.73) (width 0.2) (layer B.Cu) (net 10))
 (segment (start 148.07 111.58) (end 148.07 111.96) (width 0.2) (layer F.Cu) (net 10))
 (segment (start 149.59 111.31) (end 149.04 111.31) (width 0.2) (layer B.Cu) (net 10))
 (segment (start 150.57 112.29) (end 149.59 111.31) (width 0.2) (layer B.Cu) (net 10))
 (segment (start 151.31 114.52) (end 151.23 114.6) (width 0.13) (layer B.Cu) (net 10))
 (segment (start 151.31 113.73) (end 151.31 114.52) (width 0.2) (layer B.Cu) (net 10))
 (segment (start 148.57 111.96) (end 149.37 111.96) (width 0.2) (layer F.Cu) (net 9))
 (segment (start 149.71 111.56) (end 149.72 111.04) (width 0.2) (layer F.Cu) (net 9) (status 20))
 (segment (start 149.37 111.96) (end 149.71 111.56) (width 0.2) (layer F.Cu) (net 9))
 (segment (start 149.14 115.56) (end 148.64 115.56) (width 0.2) (layer B.Cu) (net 12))
 (segment (start 148.64 115.56) (end 148.34 115.86) (width 0.2) (layer B.Cu) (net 12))
 (segment (start 148.07 115.06) (end 148.07 115.59) (width 0.2) (layer F.Cu) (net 12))
 (segment (start 148.92 115.34) (end 148.92 114.79) (width 0.2) (layer B.Cu) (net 12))
 (segment (start 149.14 115.56) (end 148.92 115.34) (width 0.2) (layer B.Cu) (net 12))
 (via (at 149.14 115.56) (size 0.5) (drill 0.3) (layers F.Cu B.Cu) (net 12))
 (segment (start 148.93 115.77) (end 149.14 115.56) (width 0.2) (layer F.Cu) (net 12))
 (segment (start 148.25 115.77) (end 148.93 115.77) (width 0.2) (layer F.Cu) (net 12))
 (segment (start 148.07 115.59) (end 148.25 115.77) (width 0.2) (layer F.Cu) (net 12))
 (segment (start 148.92 114.79) (end 148.87 114.84) (width 0.2) (layer B.Cu) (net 12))
 (segment (start 145.14 114.41) (end 145.14 114.9) (width 0.2) (layer F.Cu) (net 1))
 (segment (start 145.14 114.9) (end 145.73 115.49) (width 0.2) (layer F.Cu) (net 1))
 (segment (start 145.14 114.41) (end 145.16 113.81) (width 0.2) (layer F.Cu) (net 1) (status 10))
 (segment (start 144.74 114.08) (end 144.74 114.7) (width 0.2) (layer B.Cu) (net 1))
 (segment (start 145.16 113.81) (end 144.74 114.08) (width 0.2) (layer B.Cu) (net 1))
 (via (at 145.16 113.81) (size 0.5) (drill 0.3) (layers F.Cu B.Cu) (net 1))
 (segment (start 144.63 115.84) (end 144.63 115.4) (width 0.2) (layer B.Cu) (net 1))
 (segment (start 144.63 115.4) (end 144.74 115.29) (width 0.2) (layer B.Cu) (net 1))
 (segment (start 144.74 115.29) (end 144.74 114.7) (width 0.2) (layer B.Cu) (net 1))
 (segment (start 146.57 115.06) (end 146.41 115.06) (width 0.2) (layer F.Cu) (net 6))
 (segment (start 145.78 114.33) (end 145.64 114.7) (width 0.2) (layer B.Cu) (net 6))
 (segment (start 145.91 114.2) (end 145.78 114.33) (width 0.2) (layer B.Cu) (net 6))
 (via (at 145.91 114.2) (size 0.5) (drill 0.3) (layers F.Cu B.Cu) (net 6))
 (segment (start 145.91 114.56) (end 145.91 114.2) (width 0.2) (layer F.Cu) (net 6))
 (segment (start 146.41 115.06) (end 145.91 114.56) (width 0.2) (layer F.Cu) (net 6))
 (segment (start 146.12 115.86) (end 146.12 115.29) (width 0.2) (layer B.Cu) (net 6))
 (segment (start 146.12 115.29) (end 146.65 114.76) (width 0.2) (layer B.Cu) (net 6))
 (segment (start 145.64 114.7) (end 145.91 114.7) (width 0.2) (layer B.Cu) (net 6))
 (segment (start 145.97 114.76) (end 146.65 114.76) (width 0.2) (layer B.Cu) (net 6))
 (segment (start 145.91 114.7) (end 145.97 114.76) (width 0.2) (layer B.Cu) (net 6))
 (segment (start 147.07 115.06) (end 147.07 115.63) (width 0.2) (layer F.Cu) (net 11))
 (segment (start 147.08 115.64) (end 147.23 115.79) (width 0.2) (layer B.Cu) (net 11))
 (via (at 147.08 115.64) (size 0.5) (drill 0.3) (layers F.Cu B.Cu) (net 11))
 (segment (start 147.07 115.63) (end 147.08 115.64) (width 0.2) (layer F.Cu) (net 11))
 (segment (start 147.23 115.79) (end 147.23 115.86) (width 0.2) (layer B.Cu) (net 11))
 (segment (start 147.23 115.86) (end 147.23 115.46) (width 0.2) (layer B.Cu) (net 11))
 (segment (start 147.23 115.46) (end 147.9 114.79) (width 0.2) (layer B.Cu) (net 11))
 (segment (start 147.9 114.79) (end 147.86 114.83) (width 0.2) (layer B.Cu) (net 11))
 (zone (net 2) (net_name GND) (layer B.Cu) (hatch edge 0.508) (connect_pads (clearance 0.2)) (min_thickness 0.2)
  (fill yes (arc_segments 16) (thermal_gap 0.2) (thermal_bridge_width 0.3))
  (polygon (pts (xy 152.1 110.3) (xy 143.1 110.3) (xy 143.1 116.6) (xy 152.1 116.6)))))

